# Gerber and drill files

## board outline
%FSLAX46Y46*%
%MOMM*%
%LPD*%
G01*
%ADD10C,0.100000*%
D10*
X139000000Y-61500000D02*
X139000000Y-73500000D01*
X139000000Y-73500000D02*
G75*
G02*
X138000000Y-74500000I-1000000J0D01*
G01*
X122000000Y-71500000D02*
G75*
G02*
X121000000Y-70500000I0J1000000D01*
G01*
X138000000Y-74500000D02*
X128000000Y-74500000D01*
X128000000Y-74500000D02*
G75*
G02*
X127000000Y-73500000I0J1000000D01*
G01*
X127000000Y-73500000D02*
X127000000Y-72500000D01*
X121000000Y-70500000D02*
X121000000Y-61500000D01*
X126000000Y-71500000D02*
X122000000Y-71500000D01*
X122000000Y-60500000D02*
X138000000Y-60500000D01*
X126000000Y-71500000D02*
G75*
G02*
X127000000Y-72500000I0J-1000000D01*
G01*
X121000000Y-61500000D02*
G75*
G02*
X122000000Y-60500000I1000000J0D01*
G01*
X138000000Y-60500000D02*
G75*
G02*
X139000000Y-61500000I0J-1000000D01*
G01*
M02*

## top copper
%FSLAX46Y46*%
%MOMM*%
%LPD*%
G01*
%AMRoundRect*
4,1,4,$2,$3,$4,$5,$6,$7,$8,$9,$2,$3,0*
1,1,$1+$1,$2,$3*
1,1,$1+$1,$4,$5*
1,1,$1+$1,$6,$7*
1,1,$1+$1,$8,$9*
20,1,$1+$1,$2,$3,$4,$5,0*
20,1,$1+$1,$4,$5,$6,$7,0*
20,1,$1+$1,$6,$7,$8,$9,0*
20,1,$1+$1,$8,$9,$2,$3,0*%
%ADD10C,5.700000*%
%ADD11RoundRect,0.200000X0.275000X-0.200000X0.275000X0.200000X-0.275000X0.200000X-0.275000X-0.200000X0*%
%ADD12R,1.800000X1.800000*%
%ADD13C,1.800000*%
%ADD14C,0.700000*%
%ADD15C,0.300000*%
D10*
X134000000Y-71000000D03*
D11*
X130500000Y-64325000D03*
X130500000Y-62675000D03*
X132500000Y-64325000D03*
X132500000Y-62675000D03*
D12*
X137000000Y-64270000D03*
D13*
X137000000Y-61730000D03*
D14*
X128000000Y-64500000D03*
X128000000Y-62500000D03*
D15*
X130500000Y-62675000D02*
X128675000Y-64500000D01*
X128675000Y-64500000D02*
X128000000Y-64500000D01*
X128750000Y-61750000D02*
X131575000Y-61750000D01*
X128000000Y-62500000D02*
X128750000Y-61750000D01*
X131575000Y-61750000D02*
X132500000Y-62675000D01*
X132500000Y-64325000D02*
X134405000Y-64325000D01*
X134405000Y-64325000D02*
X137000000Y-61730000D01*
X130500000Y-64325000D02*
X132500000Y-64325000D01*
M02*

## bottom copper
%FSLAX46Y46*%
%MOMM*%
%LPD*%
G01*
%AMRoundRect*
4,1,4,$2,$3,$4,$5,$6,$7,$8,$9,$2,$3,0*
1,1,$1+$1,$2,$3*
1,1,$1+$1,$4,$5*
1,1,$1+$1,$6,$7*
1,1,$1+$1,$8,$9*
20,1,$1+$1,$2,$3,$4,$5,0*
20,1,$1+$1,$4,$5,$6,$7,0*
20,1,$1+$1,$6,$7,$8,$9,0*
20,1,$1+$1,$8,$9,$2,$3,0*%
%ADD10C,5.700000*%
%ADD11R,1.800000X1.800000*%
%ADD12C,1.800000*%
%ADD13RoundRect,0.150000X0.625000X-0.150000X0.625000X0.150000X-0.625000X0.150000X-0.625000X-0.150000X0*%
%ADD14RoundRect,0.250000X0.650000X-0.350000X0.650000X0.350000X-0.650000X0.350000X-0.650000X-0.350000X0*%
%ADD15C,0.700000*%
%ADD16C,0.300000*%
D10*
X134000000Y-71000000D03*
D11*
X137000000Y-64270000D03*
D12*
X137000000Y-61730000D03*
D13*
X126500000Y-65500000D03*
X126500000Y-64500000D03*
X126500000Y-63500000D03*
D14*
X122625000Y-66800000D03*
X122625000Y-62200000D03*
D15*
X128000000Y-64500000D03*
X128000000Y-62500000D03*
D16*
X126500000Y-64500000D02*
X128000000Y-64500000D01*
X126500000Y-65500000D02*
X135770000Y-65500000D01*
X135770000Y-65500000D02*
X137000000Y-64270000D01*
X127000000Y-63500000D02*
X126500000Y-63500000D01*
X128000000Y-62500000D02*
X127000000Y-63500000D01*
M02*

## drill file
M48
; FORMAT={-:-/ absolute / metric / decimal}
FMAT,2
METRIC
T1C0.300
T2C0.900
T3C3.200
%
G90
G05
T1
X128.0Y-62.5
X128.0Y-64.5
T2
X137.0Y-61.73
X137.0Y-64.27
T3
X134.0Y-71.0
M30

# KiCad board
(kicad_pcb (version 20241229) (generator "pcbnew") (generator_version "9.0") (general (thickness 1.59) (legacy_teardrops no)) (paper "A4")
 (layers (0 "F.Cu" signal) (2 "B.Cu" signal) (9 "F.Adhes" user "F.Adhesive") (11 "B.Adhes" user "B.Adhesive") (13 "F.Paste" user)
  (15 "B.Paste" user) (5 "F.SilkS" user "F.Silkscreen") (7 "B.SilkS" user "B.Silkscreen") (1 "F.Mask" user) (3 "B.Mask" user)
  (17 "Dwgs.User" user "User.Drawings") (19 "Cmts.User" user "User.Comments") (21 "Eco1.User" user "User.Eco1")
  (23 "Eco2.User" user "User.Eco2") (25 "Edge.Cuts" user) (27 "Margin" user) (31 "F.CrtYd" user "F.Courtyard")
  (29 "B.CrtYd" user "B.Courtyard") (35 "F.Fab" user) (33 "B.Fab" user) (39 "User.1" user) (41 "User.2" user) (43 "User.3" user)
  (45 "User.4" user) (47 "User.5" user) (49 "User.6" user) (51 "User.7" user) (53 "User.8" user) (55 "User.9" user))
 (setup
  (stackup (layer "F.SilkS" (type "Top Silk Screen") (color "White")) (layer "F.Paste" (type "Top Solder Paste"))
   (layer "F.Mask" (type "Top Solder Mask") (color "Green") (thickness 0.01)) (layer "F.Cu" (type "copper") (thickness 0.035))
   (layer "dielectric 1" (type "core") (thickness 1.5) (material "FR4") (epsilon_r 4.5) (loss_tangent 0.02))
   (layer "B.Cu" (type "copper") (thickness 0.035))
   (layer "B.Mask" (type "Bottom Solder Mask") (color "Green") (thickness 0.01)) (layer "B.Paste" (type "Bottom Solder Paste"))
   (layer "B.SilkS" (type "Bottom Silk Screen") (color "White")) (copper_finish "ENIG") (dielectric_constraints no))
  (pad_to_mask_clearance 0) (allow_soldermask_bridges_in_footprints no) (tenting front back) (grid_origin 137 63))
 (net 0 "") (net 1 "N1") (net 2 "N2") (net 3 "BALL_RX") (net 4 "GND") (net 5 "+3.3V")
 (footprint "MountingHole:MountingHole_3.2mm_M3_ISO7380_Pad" (layer "F.Cu") (at 134 71)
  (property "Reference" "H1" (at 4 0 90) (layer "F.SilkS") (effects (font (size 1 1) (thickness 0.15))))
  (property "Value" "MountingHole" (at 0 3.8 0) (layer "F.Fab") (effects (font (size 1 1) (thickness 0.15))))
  (pad "1" thru_hole circle (at 0 0) (size 5.7 5.7) (drill 3.2) (layers "*.Cu" "*.Mask") (remove_unused_layers no) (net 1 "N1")
   (zone_connect 2)))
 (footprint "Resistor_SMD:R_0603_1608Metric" (layer "F.Cu") (at 130.5 63.5 90)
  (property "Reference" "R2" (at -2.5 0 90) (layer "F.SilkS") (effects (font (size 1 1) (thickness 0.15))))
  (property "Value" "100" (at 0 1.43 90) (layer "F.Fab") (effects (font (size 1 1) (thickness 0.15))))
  (pad "1" smd roundrect (at -0.825 0 90) (size 0.8 0.95) (layers "F.Cu" "F.Mask" "F.Paste") (roundrect_rratio 0.25) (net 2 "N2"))
  (pad "2" smd roundrect (at 0.825 0 90) (size 0.8 0.95) (layers "F.Cu" "F.Mask" "F.Paste") (roundrect_rratio 0.25) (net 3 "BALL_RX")))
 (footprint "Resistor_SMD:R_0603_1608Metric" (layer "F.Cu") (at 132.5 63.5 90)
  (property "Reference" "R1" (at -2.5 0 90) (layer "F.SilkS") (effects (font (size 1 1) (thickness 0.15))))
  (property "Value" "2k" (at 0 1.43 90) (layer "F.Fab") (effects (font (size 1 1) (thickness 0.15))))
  (pad "1" smd roundrect (at -0.825 0 90) (size 0.8 0.95) (layers "F.Cu" "F.Mask" "F.Paste") (roundrect_rratio 0.25) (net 2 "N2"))
  (pad "2" smd roundrect (at 0.825 0 90) (size 0.8 0.95) (layers "F.Cu" "F.Mask" "F.Paste") (roundrect_rratio 0.25) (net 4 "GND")))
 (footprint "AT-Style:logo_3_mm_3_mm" (layer "F.Cu") (at 129.75 68.25)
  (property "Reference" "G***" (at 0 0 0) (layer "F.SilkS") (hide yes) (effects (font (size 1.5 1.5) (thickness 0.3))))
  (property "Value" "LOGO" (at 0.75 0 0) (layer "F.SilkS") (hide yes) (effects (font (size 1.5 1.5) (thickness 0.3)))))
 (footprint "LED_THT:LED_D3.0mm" (layer "B.Cu") (at 137 64.27 90)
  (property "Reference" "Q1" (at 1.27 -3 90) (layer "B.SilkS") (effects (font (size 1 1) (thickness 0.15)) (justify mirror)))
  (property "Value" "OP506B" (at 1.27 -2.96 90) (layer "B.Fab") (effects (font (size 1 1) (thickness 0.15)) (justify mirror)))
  (pad "1" thru_hole rect (at 0 0 90) (size 1.8 1.8) (drill 0.9) (layers "*.Cu" "*.Mask") (remove_unused_layers no) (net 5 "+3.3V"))
  (pad "2" thru_hole circle (at 2.54 0 90) (size 1.8 1.8) (drill 0.9) (layers "*.Cu" "*.Mask") (remove_unused_layers no) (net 2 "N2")))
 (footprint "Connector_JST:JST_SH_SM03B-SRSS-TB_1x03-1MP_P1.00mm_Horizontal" (layer "B.Cu") (at 124.5 64.5 90)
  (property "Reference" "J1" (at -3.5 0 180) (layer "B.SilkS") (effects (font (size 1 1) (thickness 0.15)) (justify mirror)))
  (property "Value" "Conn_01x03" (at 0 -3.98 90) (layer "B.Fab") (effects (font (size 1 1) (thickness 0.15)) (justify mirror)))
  (pad "1" smd roundrect (at -1 2 90) (size 0.6 1.55) (layers "B.Cu" "B.Mask" "B.Paste") (roundrect_rratio 0.25) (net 5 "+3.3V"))
  (pad "2" smd roundrect (at 0 2 90) (size 0.6 1.55) (layers "B.Cu" "B.Mask" "B.Paste") (roundrect_rratio 0.25) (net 3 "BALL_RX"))
  (pad "3" smd roundrect (at 1 2 90) (size 0.6 1.55) (layers "B.Cu" "B.Mask" "B.Paste") (roundrect_rratio 0.25) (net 4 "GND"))
  (pad "MP" smd roundrect (at -2.3 -1.875 90) (size 1.2 1.8) (layers "B.Cu" "B.Mask" "B.Paste") (roundrect_rratio 0.208333))
  (pad "MP" smd roundrect (at 2.3 -1.875 90) (size 1.2 1.8) (layers "B.Cu" "B.Mask" "B.Paste") (roundrect_rratio 0.208333)))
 (gr_line (start 139 61.5) (end 139 73.5) (stroke (width 0.1) (type default)) (layer "Edge.Cuts"))
 (gr_arc (start 139 73.5) (mid 138.707107 74.207107) (end 138 74.5) (stroke (width 0.1) (type default)) (layer "Edge.Cuts"))
 (gr_arc (start 122 71.5) (mid 121.292893 71.207107) (end 121 70.5) (stroke (width 0.1) (type default)) (layer "Edge.Cuts"))
 (gr_line (start 138 74.5) (end 128 74.5) (stroke (width 0.1) (type default)) (layer "Edge.Cuts"))
 (gr_arc (start 128 74.5) (mid 127.292893 74.207107) (end 127 73.5) (stroke (width 0.1) (type default)) (layer "Edge.Cuts"))
 (gr_line (start 127 73.5) (end 127 72.5) (stroke (width 0.1) (type default)) (layer "Edge.Cuts"))
 (gr_line (start 121 70.5) (end 121 61.5) (stroke (width 0.1) (type default)) (layer "Edge.Cuts"))
 (gr_line (start 126 71.5) (end 122 71.5) (stroke (width 0.1) (type default)) (layer "Edge.Cuts"))
 (gr_line (start 122 60.5) (end 138 60.5) (stroke (width 0.1) (type default)) (layer "Edge.Cuts"))
 (gr_arc (start 126 71.5) (mid 126.707107 71.792893) (end 127 72.5) (stroke (width 0.1) (type default)) (layer "Edge.Cuts"))
 (gr_arc (start 121 61.5) (mid 121.292893 60.792893) (end 122 60.5) (stroke (width 0.1) (type default)) (layer "Edge.Cuts"))
 (gr_arc (start 138 60.5) (mid 138.707107 60.792893) (end 139 61.5) (stroke (width 0.1) (type default)) (layer "Edge.Cuts"))
 (segment (start 130.5 62.675) (end 128.675 64.5) (width 0.3) (layer "F.Cu") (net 3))
 (segment (start 128.675 64.5) (end 128 64.5) (width 0.3) (layer "F.Cu") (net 3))
 (via (at 128 64.5) (size 0.7) (drill 0.3) (layers "F.Cu" "B.Cu") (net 3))
 (segment (start 126.5 64.5) (end 128 64.5) (width 0.3) (layer "B.Cu") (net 3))
 (segment (start 126.5 65.5) (end 135.77 65.5) (width 0.3) (layer "B.Cu") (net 5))
 (segment (start 135.77 65.5) (end 137 64.27) (width 0.3) (layer "B.Cu") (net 5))
 (segment (start 128.75 61.75) (end 131.575 61.75) (width 0.3) (layer "F.Cu") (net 4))
 (segment (start 128 62.5) (end 128.75 61.75) (width 0.3) (layer "F.Cu") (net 4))
 (segment (start 131.575 61.75) (end 132.5 62.675) (width 0.3) (layer "F.Cu") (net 4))
 (via (at 128 62.5) (size 0.7) (drill 0.3) (layers "F.Cu" "B.Cu") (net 4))
 (segment (start 127 63.5) (end 126.5 63.5) (width 0.3) (layer "B.Cu") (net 4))
 (segment (start 128 62.5) (end 127 63.5) (width 0.3) (layer "B.Cu") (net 4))
 (segment (start 132.5 64.325) (end 134.405 64.325) (width 0.3) (layer "F.Cu") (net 2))
 (segment (start 134.405 64.325) (end 137 61.73) (width 0.3) (layer "F.Cu") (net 2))
 (segment (start 130.5 64.325) (end 132.5 64.325) (width 0.3) (layer "F.Cu") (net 2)))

